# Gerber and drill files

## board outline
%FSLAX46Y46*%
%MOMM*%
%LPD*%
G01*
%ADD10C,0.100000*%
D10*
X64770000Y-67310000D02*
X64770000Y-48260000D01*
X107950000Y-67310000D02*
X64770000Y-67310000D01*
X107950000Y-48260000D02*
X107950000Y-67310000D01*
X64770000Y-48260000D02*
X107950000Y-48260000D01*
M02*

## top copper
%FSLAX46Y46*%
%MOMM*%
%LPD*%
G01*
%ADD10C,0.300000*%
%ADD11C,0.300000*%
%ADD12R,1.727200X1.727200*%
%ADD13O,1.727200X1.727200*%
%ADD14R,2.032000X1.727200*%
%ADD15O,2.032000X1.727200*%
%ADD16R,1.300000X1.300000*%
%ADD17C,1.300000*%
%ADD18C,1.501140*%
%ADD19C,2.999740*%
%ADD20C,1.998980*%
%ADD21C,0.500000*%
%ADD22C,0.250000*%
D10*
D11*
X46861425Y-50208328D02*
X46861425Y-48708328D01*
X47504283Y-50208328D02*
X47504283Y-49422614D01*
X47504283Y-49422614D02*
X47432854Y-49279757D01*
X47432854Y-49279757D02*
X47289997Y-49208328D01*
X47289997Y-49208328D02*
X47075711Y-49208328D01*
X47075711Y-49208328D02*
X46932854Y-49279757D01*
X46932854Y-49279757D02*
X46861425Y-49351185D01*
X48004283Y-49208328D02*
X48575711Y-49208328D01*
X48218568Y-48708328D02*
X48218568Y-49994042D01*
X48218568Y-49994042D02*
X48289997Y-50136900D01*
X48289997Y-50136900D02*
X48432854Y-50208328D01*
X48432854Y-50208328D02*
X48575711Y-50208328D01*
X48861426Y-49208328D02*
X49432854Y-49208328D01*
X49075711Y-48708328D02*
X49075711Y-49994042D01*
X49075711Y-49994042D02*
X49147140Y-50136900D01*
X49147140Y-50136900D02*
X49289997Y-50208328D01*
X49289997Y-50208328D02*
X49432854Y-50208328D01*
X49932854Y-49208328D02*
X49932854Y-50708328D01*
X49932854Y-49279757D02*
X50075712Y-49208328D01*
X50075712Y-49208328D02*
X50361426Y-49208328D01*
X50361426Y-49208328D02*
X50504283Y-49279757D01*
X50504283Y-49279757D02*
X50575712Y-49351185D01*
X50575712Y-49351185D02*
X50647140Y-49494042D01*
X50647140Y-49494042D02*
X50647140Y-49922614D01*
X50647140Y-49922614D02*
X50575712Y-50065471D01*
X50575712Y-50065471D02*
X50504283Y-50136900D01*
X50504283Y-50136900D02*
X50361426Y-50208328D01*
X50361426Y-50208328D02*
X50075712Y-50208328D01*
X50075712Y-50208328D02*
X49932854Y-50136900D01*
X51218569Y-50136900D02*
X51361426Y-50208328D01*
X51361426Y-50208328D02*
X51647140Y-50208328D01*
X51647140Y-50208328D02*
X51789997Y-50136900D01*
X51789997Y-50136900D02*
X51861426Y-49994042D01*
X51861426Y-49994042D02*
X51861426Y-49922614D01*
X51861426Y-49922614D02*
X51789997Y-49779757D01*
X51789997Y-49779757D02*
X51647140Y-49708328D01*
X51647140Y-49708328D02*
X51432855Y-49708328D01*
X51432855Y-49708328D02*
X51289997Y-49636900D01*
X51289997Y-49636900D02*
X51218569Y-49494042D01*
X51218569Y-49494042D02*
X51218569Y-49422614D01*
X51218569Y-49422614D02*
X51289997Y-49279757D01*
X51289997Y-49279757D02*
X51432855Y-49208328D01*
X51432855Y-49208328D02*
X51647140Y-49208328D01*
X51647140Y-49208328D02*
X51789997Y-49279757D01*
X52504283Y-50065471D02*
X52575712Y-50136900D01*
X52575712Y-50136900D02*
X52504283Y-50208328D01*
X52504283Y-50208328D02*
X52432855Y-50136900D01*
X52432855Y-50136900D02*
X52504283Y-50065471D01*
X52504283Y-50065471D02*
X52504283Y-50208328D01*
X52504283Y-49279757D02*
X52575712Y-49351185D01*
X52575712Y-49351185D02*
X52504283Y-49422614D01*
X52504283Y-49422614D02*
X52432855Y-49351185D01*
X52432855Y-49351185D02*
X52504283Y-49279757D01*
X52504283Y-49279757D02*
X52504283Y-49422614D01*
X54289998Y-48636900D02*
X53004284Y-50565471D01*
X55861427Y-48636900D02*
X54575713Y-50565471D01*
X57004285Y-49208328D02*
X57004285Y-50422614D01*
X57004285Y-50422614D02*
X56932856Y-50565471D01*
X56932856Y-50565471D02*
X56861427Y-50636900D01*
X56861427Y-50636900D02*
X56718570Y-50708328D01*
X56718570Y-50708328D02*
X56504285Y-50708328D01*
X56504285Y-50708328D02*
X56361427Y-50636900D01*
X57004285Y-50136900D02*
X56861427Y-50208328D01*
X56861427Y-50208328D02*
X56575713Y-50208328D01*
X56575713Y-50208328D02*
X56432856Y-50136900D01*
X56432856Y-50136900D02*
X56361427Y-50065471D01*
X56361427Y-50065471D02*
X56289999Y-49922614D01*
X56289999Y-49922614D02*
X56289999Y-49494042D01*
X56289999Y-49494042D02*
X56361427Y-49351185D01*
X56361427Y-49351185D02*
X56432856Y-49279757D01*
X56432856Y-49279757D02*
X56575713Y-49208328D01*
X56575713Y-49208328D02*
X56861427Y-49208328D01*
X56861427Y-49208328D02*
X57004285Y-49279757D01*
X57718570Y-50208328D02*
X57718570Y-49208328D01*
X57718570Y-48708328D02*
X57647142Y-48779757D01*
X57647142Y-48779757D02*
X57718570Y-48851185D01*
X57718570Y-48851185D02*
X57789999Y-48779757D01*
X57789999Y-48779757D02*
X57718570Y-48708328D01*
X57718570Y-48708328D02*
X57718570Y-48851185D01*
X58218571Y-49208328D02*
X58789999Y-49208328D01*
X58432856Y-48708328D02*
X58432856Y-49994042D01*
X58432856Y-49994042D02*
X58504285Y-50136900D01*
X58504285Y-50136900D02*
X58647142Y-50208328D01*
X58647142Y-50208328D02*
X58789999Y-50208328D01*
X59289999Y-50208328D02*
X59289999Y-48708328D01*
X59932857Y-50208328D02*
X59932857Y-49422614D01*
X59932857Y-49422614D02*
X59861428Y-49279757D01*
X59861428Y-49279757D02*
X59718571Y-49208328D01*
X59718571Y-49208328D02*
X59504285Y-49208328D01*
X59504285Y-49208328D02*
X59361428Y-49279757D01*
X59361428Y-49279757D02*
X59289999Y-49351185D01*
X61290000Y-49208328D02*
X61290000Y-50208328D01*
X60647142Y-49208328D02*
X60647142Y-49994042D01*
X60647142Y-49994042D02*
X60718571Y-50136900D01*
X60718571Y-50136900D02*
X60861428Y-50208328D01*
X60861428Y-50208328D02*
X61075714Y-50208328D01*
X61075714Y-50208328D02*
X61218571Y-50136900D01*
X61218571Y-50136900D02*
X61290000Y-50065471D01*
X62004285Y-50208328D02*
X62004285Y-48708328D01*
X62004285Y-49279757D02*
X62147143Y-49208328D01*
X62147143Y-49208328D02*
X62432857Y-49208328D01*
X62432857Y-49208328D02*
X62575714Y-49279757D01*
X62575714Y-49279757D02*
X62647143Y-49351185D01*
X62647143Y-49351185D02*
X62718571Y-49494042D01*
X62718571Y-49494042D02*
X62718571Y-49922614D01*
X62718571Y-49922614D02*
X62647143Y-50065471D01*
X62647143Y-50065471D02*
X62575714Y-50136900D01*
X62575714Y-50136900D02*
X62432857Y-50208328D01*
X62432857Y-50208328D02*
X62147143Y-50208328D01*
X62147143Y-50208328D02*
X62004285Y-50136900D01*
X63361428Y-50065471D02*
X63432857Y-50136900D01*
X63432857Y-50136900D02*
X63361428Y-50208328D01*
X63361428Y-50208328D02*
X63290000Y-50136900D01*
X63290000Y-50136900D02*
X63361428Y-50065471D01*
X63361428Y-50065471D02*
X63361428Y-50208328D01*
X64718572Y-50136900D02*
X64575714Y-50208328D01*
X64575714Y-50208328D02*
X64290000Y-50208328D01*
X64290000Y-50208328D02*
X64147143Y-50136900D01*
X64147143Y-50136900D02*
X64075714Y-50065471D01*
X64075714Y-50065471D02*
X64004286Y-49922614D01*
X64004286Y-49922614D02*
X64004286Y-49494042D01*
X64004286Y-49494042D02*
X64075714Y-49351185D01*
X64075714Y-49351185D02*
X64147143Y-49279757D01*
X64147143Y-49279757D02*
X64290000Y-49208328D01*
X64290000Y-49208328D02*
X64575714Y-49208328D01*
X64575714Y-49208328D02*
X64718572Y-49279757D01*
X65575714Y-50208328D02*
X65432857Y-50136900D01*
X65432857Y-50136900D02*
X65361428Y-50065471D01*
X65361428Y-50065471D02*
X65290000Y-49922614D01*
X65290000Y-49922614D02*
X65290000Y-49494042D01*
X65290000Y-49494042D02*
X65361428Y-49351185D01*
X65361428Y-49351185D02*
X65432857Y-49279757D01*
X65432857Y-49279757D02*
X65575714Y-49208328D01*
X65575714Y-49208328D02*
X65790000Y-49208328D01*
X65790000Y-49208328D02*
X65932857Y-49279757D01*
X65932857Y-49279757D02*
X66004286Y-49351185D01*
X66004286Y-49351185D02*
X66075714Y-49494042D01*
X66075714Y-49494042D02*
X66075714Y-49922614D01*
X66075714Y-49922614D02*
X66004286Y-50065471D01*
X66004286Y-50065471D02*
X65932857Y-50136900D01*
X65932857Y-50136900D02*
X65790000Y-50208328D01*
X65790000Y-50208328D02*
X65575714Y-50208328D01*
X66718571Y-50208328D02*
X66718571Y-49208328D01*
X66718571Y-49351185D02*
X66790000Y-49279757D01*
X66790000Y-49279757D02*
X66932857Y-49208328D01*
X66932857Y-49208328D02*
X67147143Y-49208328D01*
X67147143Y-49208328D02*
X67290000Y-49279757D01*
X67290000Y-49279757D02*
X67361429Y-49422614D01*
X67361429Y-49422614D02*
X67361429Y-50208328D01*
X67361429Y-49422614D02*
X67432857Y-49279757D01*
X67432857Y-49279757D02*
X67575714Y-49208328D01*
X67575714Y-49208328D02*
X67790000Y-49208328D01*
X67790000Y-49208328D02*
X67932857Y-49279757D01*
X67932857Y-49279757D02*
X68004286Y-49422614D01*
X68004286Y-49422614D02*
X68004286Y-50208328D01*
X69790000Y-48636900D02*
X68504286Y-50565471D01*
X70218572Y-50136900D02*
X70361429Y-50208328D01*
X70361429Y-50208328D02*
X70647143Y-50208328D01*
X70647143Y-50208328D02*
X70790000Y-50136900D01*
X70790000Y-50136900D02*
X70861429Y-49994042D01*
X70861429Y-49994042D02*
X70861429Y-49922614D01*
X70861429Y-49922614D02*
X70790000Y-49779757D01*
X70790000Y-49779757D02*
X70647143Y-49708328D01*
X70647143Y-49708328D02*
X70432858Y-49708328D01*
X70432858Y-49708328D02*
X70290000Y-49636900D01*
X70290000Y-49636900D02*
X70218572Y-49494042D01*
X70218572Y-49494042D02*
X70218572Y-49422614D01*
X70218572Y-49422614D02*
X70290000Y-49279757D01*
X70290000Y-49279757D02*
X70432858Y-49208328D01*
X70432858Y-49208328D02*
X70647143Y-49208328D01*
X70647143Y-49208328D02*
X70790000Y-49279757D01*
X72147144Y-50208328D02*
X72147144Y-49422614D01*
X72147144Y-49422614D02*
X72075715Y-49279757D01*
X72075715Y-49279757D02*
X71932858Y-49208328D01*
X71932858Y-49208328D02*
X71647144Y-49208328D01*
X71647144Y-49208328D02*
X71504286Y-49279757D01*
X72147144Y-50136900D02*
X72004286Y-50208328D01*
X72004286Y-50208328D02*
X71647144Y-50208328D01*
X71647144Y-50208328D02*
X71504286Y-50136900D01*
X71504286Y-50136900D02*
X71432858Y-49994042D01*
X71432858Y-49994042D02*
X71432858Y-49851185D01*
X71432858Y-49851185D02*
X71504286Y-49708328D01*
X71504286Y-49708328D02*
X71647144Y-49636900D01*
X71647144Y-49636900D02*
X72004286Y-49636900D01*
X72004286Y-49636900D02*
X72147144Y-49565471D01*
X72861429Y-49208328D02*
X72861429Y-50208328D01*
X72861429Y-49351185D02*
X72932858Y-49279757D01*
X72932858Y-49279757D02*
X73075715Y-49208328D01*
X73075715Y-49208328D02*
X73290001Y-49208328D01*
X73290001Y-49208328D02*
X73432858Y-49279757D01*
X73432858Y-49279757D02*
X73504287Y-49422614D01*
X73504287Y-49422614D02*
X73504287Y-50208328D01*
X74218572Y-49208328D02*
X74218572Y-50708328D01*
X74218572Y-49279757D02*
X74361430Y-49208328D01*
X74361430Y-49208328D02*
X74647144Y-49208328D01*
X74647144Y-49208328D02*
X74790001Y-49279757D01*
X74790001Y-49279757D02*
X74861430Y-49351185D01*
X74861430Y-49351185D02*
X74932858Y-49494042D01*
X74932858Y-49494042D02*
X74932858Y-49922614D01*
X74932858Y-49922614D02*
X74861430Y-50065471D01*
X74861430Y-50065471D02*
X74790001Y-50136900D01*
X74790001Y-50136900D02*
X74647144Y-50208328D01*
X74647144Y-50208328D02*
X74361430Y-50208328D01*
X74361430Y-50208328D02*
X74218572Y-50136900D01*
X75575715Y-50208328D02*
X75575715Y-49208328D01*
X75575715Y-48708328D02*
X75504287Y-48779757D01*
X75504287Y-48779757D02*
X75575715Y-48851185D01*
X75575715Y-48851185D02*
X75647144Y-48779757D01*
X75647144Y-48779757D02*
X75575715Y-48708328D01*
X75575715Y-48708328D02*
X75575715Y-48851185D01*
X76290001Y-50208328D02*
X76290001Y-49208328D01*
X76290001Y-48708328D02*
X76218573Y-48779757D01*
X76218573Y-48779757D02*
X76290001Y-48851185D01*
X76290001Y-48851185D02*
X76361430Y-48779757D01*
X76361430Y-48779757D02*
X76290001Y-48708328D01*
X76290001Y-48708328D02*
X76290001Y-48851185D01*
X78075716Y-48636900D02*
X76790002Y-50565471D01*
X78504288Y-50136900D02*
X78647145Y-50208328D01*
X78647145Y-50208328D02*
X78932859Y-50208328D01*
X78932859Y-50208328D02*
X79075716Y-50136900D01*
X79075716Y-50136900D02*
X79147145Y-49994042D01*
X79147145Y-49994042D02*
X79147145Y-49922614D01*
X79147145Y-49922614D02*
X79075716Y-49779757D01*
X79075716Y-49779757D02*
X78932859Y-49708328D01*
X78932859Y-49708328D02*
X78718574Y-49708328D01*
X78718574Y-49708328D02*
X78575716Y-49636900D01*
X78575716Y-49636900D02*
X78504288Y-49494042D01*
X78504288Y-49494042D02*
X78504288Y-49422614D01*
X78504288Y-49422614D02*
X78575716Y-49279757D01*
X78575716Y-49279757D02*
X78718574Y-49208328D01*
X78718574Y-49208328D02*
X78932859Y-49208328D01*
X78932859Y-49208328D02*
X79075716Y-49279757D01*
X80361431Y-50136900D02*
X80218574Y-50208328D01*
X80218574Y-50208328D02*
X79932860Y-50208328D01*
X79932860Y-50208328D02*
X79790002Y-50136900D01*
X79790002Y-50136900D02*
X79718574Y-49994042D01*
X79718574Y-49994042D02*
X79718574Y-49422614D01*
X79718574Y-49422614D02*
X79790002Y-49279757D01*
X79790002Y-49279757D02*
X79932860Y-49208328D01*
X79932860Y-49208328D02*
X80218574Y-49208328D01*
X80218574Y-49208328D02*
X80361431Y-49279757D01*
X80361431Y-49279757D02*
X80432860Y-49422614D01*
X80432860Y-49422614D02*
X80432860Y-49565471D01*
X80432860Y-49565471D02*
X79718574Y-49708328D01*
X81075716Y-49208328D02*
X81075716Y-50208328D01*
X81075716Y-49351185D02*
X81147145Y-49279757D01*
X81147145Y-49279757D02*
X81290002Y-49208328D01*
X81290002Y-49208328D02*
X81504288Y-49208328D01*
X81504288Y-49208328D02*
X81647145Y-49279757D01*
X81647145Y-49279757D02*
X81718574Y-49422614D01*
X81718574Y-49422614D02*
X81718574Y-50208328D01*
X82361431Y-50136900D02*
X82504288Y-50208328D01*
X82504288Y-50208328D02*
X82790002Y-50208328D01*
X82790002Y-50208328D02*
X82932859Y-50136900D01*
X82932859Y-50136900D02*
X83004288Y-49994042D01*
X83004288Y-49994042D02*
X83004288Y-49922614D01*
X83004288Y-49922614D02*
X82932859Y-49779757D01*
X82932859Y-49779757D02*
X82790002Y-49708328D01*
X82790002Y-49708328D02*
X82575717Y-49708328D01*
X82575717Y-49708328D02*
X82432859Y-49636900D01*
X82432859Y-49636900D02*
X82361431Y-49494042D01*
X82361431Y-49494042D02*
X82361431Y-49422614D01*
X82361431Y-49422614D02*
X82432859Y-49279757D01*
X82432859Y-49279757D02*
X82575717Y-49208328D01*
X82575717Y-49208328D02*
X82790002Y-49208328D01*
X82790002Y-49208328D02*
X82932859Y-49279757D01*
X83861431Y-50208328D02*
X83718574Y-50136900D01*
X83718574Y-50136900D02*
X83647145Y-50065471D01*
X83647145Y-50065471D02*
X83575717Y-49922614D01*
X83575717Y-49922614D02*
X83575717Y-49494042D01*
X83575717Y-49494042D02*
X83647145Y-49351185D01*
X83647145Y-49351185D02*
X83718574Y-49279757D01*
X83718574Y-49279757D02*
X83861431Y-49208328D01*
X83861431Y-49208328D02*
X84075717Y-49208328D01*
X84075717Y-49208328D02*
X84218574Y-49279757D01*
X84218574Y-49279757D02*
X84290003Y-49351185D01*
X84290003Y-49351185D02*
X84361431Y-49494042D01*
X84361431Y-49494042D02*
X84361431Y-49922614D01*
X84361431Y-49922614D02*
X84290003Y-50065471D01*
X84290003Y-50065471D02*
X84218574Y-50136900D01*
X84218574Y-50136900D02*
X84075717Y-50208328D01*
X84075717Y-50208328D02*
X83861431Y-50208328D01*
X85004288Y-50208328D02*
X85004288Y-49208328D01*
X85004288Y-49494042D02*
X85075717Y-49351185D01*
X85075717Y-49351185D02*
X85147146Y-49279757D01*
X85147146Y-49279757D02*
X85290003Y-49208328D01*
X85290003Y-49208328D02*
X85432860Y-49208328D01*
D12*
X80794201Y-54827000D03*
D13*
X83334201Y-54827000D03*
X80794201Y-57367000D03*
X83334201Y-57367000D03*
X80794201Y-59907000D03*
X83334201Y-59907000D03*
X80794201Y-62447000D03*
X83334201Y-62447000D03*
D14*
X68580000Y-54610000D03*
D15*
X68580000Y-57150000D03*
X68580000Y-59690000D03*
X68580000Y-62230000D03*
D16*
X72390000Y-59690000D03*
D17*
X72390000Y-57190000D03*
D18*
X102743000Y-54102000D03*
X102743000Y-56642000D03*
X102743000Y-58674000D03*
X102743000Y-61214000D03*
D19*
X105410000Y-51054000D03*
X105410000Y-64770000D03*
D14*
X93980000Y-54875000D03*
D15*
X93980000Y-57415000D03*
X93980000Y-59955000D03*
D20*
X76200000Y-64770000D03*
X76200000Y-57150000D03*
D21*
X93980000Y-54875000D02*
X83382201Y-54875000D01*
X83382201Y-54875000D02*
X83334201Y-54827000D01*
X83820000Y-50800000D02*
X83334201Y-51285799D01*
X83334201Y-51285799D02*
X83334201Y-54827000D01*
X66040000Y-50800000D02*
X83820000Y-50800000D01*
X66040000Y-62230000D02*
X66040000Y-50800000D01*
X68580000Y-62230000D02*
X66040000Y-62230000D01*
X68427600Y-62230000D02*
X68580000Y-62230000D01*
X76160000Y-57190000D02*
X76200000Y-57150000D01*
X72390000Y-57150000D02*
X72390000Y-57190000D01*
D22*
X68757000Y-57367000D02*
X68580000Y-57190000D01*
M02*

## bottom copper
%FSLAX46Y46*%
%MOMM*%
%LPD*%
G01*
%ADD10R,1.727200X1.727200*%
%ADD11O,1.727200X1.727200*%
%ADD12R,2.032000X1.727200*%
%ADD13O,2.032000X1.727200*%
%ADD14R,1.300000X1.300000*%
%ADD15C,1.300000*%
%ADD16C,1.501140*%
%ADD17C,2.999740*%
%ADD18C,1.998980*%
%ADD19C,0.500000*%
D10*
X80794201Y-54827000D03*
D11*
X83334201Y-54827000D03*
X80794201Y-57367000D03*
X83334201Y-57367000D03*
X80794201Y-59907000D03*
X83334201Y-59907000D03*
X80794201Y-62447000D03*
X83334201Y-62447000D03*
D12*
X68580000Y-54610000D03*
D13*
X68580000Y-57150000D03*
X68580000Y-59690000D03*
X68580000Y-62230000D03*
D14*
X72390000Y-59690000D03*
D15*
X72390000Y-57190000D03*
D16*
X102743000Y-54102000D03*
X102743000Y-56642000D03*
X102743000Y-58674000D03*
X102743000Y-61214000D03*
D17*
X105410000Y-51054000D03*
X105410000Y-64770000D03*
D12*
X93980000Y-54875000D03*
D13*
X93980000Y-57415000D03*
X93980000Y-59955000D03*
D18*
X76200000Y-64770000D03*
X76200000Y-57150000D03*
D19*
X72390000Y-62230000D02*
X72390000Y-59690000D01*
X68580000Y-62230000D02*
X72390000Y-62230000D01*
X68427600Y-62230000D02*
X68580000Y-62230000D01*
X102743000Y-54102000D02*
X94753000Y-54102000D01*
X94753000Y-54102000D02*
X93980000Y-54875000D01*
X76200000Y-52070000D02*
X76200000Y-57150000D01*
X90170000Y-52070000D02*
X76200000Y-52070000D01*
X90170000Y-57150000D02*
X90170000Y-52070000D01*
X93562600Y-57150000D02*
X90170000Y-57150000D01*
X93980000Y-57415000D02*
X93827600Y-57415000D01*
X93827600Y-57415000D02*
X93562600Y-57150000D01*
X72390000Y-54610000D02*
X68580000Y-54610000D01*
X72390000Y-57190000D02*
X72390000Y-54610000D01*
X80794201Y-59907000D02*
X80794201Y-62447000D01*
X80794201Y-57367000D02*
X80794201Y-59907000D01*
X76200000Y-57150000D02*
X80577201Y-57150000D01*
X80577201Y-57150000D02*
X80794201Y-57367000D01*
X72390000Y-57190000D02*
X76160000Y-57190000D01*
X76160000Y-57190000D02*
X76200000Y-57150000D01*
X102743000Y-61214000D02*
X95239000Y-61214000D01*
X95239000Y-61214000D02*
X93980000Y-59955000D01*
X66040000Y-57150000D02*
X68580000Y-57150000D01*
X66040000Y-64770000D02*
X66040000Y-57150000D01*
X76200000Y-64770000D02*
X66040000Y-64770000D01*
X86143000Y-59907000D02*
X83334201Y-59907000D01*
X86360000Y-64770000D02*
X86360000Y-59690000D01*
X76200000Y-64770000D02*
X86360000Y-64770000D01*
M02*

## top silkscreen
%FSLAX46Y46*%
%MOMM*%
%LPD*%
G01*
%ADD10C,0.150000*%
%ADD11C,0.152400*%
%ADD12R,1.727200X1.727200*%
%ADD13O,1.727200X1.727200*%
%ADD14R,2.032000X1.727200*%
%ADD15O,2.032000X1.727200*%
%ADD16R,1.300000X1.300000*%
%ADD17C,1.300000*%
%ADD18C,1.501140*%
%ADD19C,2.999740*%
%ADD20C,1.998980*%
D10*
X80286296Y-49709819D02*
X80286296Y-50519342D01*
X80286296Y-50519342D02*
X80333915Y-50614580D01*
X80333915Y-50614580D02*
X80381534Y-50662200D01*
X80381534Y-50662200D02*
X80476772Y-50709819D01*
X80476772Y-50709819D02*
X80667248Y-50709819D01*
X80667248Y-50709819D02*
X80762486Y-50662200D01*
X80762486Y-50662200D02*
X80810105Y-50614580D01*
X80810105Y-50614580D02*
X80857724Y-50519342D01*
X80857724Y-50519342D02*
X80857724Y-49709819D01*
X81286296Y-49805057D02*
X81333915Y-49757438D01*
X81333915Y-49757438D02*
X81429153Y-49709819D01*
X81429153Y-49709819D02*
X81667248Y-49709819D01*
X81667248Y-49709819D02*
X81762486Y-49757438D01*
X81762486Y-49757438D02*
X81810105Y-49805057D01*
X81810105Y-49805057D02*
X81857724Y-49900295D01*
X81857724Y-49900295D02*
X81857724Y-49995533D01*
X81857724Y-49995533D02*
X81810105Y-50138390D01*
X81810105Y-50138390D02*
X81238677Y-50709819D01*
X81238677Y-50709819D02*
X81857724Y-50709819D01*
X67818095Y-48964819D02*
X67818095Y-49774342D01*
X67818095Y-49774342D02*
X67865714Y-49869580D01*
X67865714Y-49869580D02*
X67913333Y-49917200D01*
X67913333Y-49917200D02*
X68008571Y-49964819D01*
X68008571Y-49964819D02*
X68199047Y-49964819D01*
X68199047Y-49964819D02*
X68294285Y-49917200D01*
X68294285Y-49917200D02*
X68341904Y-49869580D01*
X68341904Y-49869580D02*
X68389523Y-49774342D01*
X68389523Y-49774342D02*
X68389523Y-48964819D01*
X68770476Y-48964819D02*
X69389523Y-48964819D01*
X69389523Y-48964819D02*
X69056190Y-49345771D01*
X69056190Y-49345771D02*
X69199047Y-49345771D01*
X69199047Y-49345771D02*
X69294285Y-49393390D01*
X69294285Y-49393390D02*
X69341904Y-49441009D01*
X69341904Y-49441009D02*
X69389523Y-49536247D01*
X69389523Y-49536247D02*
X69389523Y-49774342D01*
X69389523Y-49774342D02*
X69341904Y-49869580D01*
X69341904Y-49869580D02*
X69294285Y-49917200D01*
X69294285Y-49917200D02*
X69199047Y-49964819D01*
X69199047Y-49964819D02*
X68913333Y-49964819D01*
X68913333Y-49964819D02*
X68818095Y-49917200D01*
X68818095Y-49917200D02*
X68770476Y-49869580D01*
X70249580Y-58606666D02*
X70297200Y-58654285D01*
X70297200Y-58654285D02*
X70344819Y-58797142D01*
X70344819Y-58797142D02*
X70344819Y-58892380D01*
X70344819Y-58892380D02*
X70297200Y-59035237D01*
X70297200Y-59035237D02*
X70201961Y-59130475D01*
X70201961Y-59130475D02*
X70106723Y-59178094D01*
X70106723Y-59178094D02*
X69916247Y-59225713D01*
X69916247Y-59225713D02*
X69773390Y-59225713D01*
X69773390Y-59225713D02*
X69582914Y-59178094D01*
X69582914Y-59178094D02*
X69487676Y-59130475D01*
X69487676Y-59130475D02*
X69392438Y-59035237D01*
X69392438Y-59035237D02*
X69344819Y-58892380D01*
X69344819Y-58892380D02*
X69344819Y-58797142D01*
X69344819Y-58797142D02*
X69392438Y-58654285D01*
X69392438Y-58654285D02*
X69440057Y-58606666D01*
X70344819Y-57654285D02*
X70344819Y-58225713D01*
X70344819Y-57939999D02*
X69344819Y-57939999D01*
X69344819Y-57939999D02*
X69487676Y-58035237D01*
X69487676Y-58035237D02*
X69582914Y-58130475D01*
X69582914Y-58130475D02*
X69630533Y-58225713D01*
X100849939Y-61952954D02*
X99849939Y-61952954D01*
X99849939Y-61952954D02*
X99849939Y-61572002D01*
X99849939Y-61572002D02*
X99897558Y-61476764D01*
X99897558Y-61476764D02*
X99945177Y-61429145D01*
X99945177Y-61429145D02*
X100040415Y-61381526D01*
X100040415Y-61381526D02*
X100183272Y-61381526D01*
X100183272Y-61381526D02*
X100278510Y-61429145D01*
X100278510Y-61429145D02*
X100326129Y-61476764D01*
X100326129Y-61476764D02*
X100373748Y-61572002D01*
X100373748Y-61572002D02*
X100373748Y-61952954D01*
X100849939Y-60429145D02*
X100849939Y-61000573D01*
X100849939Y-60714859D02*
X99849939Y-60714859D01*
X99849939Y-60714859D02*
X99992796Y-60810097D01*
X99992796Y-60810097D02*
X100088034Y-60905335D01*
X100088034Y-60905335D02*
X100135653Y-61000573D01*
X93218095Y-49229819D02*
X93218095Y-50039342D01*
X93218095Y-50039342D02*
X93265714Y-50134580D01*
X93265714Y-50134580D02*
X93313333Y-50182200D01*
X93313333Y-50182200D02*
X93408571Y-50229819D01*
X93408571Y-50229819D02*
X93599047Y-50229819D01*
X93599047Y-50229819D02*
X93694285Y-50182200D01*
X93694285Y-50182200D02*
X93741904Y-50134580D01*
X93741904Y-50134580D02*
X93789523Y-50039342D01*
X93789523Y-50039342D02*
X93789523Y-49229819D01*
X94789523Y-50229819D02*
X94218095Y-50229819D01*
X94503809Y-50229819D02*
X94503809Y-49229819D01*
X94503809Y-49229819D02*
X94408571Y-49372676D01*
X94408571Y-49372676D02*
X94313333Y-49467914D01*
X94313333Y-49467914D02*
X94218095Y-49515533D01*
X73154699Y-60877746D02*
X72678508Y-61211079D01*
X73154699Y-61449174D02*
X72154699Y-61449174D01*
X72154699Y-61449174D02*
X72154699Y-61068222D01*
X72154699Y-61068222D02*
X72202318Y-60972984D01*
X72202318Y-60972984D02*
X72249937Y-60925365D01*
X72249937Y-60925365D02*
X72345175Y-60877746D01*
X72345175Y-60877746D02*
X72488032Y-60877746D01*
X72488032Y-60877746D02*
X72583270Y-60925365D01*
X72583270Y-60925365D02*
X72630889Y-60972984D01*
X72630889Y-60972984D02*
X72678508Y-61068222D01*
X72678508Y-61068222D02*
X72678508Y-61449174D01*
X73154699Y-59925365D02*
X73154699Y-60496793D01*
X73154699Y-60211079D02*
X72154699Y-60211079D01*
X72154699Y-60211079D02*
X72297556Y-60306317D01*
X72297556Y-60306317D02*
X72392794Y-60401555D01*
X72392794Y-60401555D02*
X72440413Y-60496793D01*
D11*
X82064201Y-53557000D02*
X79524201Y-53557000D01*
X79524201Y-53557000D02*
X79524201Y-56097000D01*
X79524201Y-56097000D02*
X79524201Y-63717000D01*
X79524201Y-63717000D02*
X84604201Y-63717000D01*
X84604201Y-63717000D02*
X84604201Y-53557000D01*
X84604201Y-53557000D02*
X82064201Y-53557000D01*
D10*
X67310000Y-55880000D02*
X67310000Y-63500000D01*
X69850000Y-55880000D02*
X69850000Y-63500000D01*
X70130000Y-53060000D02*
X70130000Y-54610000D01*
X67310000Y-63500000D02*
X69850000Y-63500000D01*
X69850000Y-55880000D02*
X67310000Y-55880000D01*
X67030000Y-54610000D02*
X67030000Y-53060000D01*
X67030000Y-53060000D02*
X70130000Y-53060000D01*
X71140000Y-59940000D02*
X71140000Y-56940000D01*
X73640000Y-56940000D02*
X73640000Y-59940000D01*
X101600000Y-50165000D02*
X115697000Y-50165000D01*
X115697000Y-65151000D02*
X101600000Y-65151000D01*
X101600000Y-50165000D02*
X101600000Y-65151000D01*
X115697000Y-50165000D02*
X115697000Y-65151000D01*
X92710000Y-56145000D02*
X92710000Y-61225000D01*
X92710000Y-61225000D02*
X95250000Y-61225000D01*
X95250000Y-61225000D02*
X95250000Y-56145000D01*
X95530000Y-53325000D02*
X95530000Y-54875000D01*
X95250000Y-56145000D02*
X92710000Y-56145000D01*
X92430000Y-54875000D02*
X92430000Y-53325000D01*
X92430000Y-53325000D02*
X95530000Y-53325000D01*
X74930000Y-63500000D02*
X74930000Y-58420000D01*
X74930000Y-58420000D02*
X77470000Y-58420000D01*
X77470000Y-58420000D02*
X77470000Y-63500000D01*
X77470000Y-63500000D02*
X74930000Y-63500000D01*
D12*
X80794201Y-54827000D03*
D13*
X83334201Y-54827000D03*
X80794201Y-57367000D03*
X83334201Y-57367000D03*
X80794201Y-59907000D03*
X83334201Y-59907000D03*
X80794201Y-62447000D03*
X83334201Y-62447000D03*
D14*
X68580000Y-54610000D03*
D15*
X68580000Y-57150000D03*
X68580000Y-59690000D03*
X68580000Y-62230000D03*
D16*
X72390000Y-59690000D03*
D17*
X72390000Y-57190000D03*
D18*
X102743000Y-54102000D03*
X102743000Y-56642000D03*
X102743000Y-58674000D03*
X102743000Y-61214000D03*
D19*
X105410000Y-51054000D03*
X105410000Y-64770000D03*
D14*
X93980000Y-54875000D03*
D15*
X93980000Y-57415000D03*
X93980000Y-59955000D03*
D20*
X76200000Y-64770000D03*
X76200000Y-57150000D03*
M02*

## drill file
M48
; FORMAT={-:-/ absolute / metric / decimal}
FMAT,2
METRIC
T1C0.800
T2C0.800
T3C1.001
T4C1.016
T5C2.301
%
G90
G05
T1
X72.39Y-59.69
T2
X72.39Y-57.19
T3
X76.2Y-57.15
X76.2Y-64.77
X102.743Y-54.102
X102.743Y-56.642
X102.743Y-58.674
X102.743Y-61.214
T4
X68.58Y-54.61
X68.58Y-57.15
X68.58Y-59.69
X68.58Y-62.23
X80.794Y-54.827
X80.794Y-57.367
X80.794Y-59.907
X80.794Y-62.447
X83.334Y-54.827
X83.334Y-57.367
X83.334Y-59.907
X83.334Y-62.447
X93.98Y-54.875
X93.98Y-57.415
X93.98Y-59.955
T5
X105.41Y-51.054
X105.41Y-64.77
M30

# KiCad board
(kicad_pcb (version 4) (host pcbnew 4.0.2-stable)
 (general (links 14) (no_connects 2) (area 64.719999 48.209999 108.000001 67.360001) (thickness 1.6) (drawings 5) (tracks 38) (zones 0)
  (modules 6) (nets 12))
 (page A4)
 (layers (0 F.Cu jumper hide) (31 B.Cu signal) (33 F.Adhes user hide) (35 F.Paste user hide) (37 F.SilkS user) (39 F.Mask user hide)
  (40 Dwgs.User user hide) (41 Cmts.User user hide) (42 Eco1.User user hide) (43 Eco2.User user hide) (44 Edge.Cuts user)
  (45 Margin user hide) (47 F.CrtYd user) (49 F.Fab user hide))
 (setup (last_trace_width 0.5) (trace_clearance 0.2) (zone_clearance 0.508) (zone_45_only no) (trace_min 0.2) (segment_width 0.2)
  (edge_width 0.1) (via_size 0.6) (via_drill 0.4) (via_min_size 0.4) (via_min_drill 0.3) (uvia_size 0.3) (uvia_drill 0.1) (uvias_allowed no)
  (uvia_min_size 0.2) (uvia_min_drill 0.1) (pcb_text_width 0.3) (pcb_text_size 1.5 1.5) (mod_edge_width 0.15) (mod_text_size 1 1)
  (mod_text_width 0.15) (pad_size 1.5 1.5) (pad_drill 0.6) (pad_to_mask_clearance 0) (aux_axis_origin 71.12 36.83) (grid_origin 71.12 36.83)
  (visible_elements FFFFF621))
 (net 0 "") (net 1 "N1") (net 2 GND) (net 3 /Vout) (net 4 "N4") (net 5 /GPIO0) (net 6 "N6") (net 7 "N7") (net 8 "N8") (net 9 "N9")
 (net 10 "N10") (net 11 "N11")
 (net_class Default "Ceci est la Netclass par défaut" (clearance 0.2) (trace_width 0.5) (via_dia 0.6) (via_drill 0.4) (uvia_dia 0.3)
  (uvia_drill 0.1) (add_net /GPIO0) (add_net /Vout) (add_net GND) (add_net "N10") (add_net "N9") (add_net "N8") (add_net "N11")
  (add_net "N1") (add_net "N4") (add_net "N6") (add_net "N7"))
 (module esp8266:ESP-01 (layer F.Cu) (at 80.794201 54.827)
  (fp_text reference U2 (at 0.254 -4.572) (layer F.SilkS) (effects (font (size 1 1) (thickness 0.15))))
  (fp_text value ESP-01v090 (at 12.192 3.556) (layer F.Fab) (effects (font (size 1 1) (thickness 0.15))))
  (fp_line (start 1.27 -1.27) (end -1.27 -1.27) (layer F.SilkS) (width 0.1524))
  (fp_line (start -1.27 -1.27) (end -1.27 1.27) (layer F.SilkS) (width 0.1524))
  (fp_line (start -1.27 1.27) (end -1.27 8.89) (layer F.SilkS) (width 0.1524))
  (fp_line (start -1.27 8.89) (end 3.81 8.89) (layer F.SilkS) (width 0.1524))
  (fp_line (start 3.81 8.89) (end 3.81 -1.27) (layer F.SilkS) (width 0.1524))
  (fp_line (start 3.81 -1.27) (end 1.27 -1.27) (layer F.SilkS) (width 0.1524))
  (pad 1 thru_hole rect (at 0 0) (size 1.7272 1.7272) (drill 1.016) (layers *.Cu *.Mask F.SilkS) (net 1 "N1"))
  (pad 2 thru_hole oval (at 2.54 0) (size 1.7272 1.7272) (drill 1.016) (layers *.Cu *.Mask F.SilkS) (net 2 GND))
  (pad 3 thru_hole oval (at 0 2.54) (size 1.7272 1.7272) (drill 1.016) (layers *.Cu *.Mask F.SilkS) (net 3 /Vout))
  (pad 4 thru_hole oval (at 2.54 2.54) (size 1.7272 1.7272) (drill 1.016) (layers *.Cu *.Mask F.SilkS) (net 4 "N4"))
  (pad 5 thru_hole oval (at 0 5.08) (size 1.7272 1.7272) (drill 1.016) (layers *.Cu *.Mask F.SilkS) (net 3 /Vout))
  (pad 6 thru_hole oval (at 2.54 5.08) (size 1.7272 1.7272) (drill 1.016) (layers *.Cu *.Mask F.SilkS) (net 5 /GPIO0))
  (pad 7 thru_hole oval (at 0 7.62) (size 1.7272 1.7272) (drill 1.016) (layers *.Cu *.Mask F.SilkS) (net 3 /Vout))
  (pad 8 thru_hole oval (at 2.54 7.62) (size 1.7272 1.7272) (drill 1.016) (layers *.Cu *.Mask F.SilkS) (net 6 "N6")))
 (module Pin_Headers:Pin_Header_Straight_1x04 (layer F.Cu) (at 68.58 54.61)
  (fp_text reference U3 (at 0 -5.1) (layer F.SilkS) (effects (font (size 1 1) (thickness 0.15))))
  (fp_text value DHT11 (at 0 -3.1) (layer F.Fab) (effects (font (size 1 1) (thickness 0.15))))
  (fp_line (start -1.27 1.27) (end -1.27 8.89) (layer F.SilkS) (width 0.15))
  (fp_line (start 1.27 1.27) (end 1.27 8.89) (layer F.SilkS) (width 0.15))
  (fp_line (start 1.55 -1.55) (end 1.55 0) (layer F.SilkS) (width 0.15))
  (fp_line (start -1.27 8.89) (end 1.27 8.89) (layer F.SilkS) (width 0.15))
  (fp_line (start 1.27 1.27) (end -1.27 1.27) (layer F.SilkS) (width 0.15))
  (fp_line (start -1.55 0) (end -1.55 -1.55) (layer F.SilkS) (width 0.15))
  (fp_line (start -1.55 -1.55) (end 1.55 -1.55) (layer F.SilkS) (width 0.15))
  (pad 1 thru_hole rect (at 0 0) (size 2.032 1.7272) (drill 1.016) (layers *.Cu *.Mask F.SilkS) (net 3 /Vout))
  (pad 2 thru_hole oval (at 0 2.54) (size 2.032 1.7272) (drill 1.016) (layers *.Cu *.Mask F.SilkS) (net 5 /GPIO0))
  (pad 3 thru_hole oval (at 0 5.08) (size 2.032 1.7272) (drill 1.016) (layers *.Cu *.Mask F.SilkS) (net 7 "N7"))
  (pad 4 thru_hole oval (at 0 7.62) (size 2.032 1.7272) (drill 1.016) (layers *.Cu *.Mask F.SilkS) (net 2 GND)))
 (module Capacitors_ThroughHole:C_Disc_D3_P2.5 (layer F.Cu) (at 72.39 59.69 90)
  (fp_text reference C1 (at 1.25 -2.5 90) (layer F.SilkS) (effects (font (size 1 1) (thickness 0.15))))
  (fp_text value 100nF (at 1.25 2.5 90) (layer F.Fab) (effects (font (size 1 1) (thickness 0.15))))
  (fp_line (start -0.25 -1.25) (end 2.75 -1.25) (layer F.SilkS) (width 0.15))
  (fp_line (start 2.75 1.25) (end -0.25 1.25) (layer F.SilkS) (width 0.15))
  (pad 1 thru_hole rect (at 0 0 90) (size 1.3 1.3) (drill 0.8) (layers *.Cu *.Mask F.SilkS) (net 2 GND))
  (pad 2 thru_hole circle (at 2.5 0 90) (size 1.3 1.3) (drill 0.8001) (layers *.Cu *.Mask F.SilkS) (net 3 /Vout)))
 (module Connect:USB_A (layer F.Cu) (at 102.74512 61.21486 90)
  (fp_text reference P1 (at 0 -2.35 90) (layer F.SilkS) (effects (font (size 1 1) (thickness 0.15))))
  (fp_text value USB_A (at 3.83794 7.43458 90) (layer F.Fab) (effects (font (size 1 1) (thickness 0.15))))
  (fp_line (start 11.04986 -1.14512) (end 11.04986 12.95188) (layer F.SilkS) (width 0.15))
  (fp_line (start -3.93614 12.95188) (end -3.93614 -1.14512) (layer F.SilkS) (width 0.15))
  (fp_line (start 11.04986 -1.14512) (end -3.93614 -1.14512) (layer F.SilkS) (width 0.15))
  (fp_line (start 11.04986 12.95188) (end -3.93614 12.95188) (layer F.SilkS) (width 0.15))
  (pad 4 thru_hole circle (at 7.11286 -0.00212) (size 1.50114 1.50114) (drill 1.00076) (layers *.Cu *.Mask F.SilkS) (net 2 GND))
  (pad 3 thru_hole circle (at 4.57286 -0.00212) (size 1.50114 1.50114) (drill 1.00076) (layers *.Cu *.Mask F.SilkS) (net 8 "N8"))
  (pad 2 thru_hole circle (at 2.54086 -0.00212) (size 1.50114 1.50114) (drill 1.00076) (layers *.Cu *.Mask F.SilkS) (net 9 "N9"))
  (pad 1 thru_hole circle (at 0.00086 -0.00212) (size 1.50114 1.50114) (drill 1.00076) (layers *.Cu *.Mask F.SilkS) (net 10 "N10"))
  (pad 5 thru_hole circle (at 10.16086 2.66488) (size 2.99974 2.99974) (drill 2.30124) (layers *.Cu *.Mask F.SilkS) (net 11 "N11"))
  (pad 5 thru_hole circle (at -3.55514 2.66488) (size 2.99974 2.99974) (drill 2.30124) (layers *.Cu *.Mask F.SilkS) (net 11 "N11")))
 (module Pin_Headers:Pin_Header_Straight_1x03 (layer F.Cu) (at 93.98 54.875)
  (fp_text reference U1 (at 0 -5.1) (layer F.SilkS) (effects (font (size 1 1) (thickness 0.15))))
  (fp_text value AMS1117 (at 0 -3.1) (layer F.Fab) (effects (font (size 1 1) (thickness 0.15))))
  (fp_line (start -1.27 1.27) (end -1.27 6.35) (layer F.SilkS) (width 0.15))
  (fp_line (start -1.27 6.35) (end 1.27 6.35) (layer F.SilkS) (width 0.15))
  (fp_line (start 1.27 6.35) (end 1.27 1.27) (layer F.SilkS) (width 0.15))
  (fp_line (start 1.55 -1.55) (end 1.55 0) (layer F.SilkS) (width 0.15))
  (fp_line (start 1.27 1.27) (end -1.27 1.27) (layer F.SilkS) (width 0.15))
  (fp_line (start -1.55 0) (end -1.55 -1.55) (layer F.SilkS) (width 0.15))
  (fp_line (start -1.55 -1.55) (end 1.55 -1.55) (layer F.SilkS) (width 0.15))
  (pad 1 thru_hole rect (at 0 0) (size 2.032 1.7272) (drill 1.016) (layers *.Cu *.Mask F.SilkS) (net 2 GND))
  (pad 2 thru_hole oval (at 0 2.54) (size 2.032 1.7272) (drill 1.016) (layers *.Cu *.Mask F.SilkS) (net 3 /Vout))
  (pad 3 thru_hole oval (at 0 5.08) (size 2.032 1.7272) (drill 1.016) (layers *.Cu *.Mask F.SilkS) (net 10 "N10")))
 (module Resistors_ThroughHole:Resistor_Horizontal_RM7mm (layer F.Cu) (at 76.2 64.77 90)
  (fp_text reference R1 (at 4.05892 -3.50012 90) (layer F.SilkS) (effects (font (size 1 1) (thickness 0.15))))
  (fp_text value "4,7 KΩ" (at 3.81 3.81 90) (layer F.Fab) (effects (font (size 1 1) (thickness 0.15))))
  (fp_line (start 1.27 -1.27) (end 6.35 -1.27) (layer F.SilkS) (width 0.15))
  (fp_line (start 6.35 -1.27) (end 6.35 1.27) (layer F.SilkS) (width 0.15))
  (fp_line (start 6.35 1.27) (end 1.27 1.27) (layer F.SilkS) (width 0.15))
  (fp_line (start 1.27 1.27) (end 1.27 -1.27) (layer F.SilkS) (width 0.15))
  (pad 1 thru_hole circle (at 0 0 90) (size 1.99898 1.99898) (drill 1.00076) (layers *.Cu *.SilkS *.Mask) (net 5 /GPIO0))
  (pad 2 thru_hole circle (at 7.62 0 90) (size 1.99898 1.99898) (drill 1.00076) (layers *.Cu *.SilkS *.Mask) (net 3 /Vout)))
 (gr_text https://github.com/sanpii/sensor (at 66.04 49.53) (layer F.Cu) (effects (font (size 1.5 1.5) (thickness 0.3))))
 (gr_line (start 64.77 67.31) (end 64.77 48.26) (layer Edge.Cuts) (width 0.1))
 (gr_line (start 107.95 67.31) (end 64.77 67.31) (layer Edge.Cuts) (width 0.1))
 (gr_line (start 107.95 48.26) (end 107.95 67.31) (layer Edge.Cuts) (width 0.1))
 (gr_line (start 64.77 48.26) (end 107.95 48.26) (layer Edge.Cuts) (width 0.1))
 (segment (start 93.98 54.875) (end 83.382201 54.875) (width 0.5) (layer F.Cu) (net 2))
 (segment (start 83.382201 54.875) (end 83.334201 54.827) (width 0.5) (layer F.Cu) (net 2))
 (segment (start 83.82 50.8) (end 83.334201 51.285799) (width 0.5) (layer F.Cu) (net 2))
 (segment (start 83.334201 51.285799) (end 83.334201 54.827) (width 0.5) (layer F.Cu) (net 2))
 (segment (start 66.04 50.8) (end 83.82 50.8) (width 0.5) (layer F.Cu) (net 2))
 (segment (start 66.04 62.23) (end 66.04 50.8) (width 0.5) (layer F.Cu) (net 2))
 (segment (start 68.58 62.23) (end 66.04 62.23) (width 0.5) (layer F.Cu) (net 2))
 (segment (start 68.4276 62.23) (end 68.58 62.23) (width 0.5) (layer F.Cu) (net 2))
 (segment (start 72.39 62.23) (end 72.39 59.69) (width 0.5) (layer B.Cu) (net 2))
 (segment (start 68.58 62.23) (end 72.39 62.23) (width 0.5) (layer B.Cu) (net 2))
 (segment (start 68.4276 62.23) (end 68.58 62.23) (width 0.5) (layer B.Cu) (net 2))
 (segment (start 102.743 54.102) (end 94.753 54.102) (width 0.5) (layer B.Cu) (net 2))
 (segment (start 94.753 54.102) (end 93.98 54.875) (width 0.5) (layer B.Cu) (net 2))
 (segment (start 76.2 52.07) (end 76.2 57.15) (width 0.5) (layer B.Cu) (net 3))
 (segment (start 90.17 52.07) (end 76.2 52.07) (width 0.5) (layer B.Cu) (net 3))
 (segment (start 90.17 57.15) (end 90.17 52.07) (width 0.5) (layer B.Cu) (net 3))
 (segment (start 93.5626 57.15) (end 90.17 57.15) (width 0.5) (layer B.Cu) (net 3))
 (segment (start 93.98 57.415) (end 93.8276 57.415) (width 0.5) (layer B.Cu) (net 3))
 (segment (start 93.8276 57.415) (end 93.5626 57.15) (width 0.5) (layer B.Cu) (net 3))
 (segment (start 72.39 54.61) (end 68.58 54.61) (width 0.5) (layer B.Cu) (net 3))
 (segment (start 72.39 57.19) (end 72.39 54.61) (width 0.5) (layer B.Cu) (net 3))
 (segment (start 80.794201 59.907) (end 80.794201 62.447) (width 0.5) (layer B.Cu) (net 3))
 (segment (start 80.794201 57.367) (end 80.794201 59.907) (width 0.5) (layer B.Cu) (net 3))
 (segment (start 76.2 57.15) (end 80.577201 57.15) (width 0.5) (layer B.Cu) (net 3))
 (segment (start 80.577201 57.15) (end 80.794201 57.367) (width 0.5) (layer B.Cu) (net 3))
 (segment (start 72.39 57.19) (end 76.16 57.19) (width 0.5) (layer B.Cu) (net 3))
 (segment (start 76.16 57.19) (end 76.2 57.15) (width 0.5) (layer B.Cu) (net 3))
 (segment (start 76.16 57.19) (end 76.2 57.15) (width 0.5) (layer F.Cu) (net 3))
 (segment (start 72.39 57.15) (end 72.39 57.19) (width 0.5) (layer F.Cu) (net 3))
 (segment (start 102.743 61.214) (end 95.239 61.214) (width 0.5) (layer B.Cu) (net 10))
 (segment (start 95.239 61.214) (end 93.98 59.955) (width 0.5) (layer B.Cu) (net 10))
 (segment (start 66.04 57.15) (end 68.58 57.15) (width 0.5) (layer B.Cu) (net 5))
 (segment (start 66.04 64.77) (end 66.04 57.15) (width 0.5) (layer B.Cu) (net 5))
 (segment (start 76.2 64.77) (end 66.04 64.77) (width 0.5) (layer B.Cu) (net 5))
 (segment (start 86.143 59.907) (end 83.334201 59.907) (width 0.5) (layer B.Cu) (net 5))
 (segment (start 86.36 64.77) (end 86.36 59.69) (width 0.5) (layer B.Cu) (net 5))
 (segment (start 76.2 64.77) (end 86.36 64.77) (width 0.5) (layer B.Cu) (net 5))
 (segment (start 68.757 57.367) (end 68.58 57.19) (width 0.25) (layer F.Cu) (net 5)))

